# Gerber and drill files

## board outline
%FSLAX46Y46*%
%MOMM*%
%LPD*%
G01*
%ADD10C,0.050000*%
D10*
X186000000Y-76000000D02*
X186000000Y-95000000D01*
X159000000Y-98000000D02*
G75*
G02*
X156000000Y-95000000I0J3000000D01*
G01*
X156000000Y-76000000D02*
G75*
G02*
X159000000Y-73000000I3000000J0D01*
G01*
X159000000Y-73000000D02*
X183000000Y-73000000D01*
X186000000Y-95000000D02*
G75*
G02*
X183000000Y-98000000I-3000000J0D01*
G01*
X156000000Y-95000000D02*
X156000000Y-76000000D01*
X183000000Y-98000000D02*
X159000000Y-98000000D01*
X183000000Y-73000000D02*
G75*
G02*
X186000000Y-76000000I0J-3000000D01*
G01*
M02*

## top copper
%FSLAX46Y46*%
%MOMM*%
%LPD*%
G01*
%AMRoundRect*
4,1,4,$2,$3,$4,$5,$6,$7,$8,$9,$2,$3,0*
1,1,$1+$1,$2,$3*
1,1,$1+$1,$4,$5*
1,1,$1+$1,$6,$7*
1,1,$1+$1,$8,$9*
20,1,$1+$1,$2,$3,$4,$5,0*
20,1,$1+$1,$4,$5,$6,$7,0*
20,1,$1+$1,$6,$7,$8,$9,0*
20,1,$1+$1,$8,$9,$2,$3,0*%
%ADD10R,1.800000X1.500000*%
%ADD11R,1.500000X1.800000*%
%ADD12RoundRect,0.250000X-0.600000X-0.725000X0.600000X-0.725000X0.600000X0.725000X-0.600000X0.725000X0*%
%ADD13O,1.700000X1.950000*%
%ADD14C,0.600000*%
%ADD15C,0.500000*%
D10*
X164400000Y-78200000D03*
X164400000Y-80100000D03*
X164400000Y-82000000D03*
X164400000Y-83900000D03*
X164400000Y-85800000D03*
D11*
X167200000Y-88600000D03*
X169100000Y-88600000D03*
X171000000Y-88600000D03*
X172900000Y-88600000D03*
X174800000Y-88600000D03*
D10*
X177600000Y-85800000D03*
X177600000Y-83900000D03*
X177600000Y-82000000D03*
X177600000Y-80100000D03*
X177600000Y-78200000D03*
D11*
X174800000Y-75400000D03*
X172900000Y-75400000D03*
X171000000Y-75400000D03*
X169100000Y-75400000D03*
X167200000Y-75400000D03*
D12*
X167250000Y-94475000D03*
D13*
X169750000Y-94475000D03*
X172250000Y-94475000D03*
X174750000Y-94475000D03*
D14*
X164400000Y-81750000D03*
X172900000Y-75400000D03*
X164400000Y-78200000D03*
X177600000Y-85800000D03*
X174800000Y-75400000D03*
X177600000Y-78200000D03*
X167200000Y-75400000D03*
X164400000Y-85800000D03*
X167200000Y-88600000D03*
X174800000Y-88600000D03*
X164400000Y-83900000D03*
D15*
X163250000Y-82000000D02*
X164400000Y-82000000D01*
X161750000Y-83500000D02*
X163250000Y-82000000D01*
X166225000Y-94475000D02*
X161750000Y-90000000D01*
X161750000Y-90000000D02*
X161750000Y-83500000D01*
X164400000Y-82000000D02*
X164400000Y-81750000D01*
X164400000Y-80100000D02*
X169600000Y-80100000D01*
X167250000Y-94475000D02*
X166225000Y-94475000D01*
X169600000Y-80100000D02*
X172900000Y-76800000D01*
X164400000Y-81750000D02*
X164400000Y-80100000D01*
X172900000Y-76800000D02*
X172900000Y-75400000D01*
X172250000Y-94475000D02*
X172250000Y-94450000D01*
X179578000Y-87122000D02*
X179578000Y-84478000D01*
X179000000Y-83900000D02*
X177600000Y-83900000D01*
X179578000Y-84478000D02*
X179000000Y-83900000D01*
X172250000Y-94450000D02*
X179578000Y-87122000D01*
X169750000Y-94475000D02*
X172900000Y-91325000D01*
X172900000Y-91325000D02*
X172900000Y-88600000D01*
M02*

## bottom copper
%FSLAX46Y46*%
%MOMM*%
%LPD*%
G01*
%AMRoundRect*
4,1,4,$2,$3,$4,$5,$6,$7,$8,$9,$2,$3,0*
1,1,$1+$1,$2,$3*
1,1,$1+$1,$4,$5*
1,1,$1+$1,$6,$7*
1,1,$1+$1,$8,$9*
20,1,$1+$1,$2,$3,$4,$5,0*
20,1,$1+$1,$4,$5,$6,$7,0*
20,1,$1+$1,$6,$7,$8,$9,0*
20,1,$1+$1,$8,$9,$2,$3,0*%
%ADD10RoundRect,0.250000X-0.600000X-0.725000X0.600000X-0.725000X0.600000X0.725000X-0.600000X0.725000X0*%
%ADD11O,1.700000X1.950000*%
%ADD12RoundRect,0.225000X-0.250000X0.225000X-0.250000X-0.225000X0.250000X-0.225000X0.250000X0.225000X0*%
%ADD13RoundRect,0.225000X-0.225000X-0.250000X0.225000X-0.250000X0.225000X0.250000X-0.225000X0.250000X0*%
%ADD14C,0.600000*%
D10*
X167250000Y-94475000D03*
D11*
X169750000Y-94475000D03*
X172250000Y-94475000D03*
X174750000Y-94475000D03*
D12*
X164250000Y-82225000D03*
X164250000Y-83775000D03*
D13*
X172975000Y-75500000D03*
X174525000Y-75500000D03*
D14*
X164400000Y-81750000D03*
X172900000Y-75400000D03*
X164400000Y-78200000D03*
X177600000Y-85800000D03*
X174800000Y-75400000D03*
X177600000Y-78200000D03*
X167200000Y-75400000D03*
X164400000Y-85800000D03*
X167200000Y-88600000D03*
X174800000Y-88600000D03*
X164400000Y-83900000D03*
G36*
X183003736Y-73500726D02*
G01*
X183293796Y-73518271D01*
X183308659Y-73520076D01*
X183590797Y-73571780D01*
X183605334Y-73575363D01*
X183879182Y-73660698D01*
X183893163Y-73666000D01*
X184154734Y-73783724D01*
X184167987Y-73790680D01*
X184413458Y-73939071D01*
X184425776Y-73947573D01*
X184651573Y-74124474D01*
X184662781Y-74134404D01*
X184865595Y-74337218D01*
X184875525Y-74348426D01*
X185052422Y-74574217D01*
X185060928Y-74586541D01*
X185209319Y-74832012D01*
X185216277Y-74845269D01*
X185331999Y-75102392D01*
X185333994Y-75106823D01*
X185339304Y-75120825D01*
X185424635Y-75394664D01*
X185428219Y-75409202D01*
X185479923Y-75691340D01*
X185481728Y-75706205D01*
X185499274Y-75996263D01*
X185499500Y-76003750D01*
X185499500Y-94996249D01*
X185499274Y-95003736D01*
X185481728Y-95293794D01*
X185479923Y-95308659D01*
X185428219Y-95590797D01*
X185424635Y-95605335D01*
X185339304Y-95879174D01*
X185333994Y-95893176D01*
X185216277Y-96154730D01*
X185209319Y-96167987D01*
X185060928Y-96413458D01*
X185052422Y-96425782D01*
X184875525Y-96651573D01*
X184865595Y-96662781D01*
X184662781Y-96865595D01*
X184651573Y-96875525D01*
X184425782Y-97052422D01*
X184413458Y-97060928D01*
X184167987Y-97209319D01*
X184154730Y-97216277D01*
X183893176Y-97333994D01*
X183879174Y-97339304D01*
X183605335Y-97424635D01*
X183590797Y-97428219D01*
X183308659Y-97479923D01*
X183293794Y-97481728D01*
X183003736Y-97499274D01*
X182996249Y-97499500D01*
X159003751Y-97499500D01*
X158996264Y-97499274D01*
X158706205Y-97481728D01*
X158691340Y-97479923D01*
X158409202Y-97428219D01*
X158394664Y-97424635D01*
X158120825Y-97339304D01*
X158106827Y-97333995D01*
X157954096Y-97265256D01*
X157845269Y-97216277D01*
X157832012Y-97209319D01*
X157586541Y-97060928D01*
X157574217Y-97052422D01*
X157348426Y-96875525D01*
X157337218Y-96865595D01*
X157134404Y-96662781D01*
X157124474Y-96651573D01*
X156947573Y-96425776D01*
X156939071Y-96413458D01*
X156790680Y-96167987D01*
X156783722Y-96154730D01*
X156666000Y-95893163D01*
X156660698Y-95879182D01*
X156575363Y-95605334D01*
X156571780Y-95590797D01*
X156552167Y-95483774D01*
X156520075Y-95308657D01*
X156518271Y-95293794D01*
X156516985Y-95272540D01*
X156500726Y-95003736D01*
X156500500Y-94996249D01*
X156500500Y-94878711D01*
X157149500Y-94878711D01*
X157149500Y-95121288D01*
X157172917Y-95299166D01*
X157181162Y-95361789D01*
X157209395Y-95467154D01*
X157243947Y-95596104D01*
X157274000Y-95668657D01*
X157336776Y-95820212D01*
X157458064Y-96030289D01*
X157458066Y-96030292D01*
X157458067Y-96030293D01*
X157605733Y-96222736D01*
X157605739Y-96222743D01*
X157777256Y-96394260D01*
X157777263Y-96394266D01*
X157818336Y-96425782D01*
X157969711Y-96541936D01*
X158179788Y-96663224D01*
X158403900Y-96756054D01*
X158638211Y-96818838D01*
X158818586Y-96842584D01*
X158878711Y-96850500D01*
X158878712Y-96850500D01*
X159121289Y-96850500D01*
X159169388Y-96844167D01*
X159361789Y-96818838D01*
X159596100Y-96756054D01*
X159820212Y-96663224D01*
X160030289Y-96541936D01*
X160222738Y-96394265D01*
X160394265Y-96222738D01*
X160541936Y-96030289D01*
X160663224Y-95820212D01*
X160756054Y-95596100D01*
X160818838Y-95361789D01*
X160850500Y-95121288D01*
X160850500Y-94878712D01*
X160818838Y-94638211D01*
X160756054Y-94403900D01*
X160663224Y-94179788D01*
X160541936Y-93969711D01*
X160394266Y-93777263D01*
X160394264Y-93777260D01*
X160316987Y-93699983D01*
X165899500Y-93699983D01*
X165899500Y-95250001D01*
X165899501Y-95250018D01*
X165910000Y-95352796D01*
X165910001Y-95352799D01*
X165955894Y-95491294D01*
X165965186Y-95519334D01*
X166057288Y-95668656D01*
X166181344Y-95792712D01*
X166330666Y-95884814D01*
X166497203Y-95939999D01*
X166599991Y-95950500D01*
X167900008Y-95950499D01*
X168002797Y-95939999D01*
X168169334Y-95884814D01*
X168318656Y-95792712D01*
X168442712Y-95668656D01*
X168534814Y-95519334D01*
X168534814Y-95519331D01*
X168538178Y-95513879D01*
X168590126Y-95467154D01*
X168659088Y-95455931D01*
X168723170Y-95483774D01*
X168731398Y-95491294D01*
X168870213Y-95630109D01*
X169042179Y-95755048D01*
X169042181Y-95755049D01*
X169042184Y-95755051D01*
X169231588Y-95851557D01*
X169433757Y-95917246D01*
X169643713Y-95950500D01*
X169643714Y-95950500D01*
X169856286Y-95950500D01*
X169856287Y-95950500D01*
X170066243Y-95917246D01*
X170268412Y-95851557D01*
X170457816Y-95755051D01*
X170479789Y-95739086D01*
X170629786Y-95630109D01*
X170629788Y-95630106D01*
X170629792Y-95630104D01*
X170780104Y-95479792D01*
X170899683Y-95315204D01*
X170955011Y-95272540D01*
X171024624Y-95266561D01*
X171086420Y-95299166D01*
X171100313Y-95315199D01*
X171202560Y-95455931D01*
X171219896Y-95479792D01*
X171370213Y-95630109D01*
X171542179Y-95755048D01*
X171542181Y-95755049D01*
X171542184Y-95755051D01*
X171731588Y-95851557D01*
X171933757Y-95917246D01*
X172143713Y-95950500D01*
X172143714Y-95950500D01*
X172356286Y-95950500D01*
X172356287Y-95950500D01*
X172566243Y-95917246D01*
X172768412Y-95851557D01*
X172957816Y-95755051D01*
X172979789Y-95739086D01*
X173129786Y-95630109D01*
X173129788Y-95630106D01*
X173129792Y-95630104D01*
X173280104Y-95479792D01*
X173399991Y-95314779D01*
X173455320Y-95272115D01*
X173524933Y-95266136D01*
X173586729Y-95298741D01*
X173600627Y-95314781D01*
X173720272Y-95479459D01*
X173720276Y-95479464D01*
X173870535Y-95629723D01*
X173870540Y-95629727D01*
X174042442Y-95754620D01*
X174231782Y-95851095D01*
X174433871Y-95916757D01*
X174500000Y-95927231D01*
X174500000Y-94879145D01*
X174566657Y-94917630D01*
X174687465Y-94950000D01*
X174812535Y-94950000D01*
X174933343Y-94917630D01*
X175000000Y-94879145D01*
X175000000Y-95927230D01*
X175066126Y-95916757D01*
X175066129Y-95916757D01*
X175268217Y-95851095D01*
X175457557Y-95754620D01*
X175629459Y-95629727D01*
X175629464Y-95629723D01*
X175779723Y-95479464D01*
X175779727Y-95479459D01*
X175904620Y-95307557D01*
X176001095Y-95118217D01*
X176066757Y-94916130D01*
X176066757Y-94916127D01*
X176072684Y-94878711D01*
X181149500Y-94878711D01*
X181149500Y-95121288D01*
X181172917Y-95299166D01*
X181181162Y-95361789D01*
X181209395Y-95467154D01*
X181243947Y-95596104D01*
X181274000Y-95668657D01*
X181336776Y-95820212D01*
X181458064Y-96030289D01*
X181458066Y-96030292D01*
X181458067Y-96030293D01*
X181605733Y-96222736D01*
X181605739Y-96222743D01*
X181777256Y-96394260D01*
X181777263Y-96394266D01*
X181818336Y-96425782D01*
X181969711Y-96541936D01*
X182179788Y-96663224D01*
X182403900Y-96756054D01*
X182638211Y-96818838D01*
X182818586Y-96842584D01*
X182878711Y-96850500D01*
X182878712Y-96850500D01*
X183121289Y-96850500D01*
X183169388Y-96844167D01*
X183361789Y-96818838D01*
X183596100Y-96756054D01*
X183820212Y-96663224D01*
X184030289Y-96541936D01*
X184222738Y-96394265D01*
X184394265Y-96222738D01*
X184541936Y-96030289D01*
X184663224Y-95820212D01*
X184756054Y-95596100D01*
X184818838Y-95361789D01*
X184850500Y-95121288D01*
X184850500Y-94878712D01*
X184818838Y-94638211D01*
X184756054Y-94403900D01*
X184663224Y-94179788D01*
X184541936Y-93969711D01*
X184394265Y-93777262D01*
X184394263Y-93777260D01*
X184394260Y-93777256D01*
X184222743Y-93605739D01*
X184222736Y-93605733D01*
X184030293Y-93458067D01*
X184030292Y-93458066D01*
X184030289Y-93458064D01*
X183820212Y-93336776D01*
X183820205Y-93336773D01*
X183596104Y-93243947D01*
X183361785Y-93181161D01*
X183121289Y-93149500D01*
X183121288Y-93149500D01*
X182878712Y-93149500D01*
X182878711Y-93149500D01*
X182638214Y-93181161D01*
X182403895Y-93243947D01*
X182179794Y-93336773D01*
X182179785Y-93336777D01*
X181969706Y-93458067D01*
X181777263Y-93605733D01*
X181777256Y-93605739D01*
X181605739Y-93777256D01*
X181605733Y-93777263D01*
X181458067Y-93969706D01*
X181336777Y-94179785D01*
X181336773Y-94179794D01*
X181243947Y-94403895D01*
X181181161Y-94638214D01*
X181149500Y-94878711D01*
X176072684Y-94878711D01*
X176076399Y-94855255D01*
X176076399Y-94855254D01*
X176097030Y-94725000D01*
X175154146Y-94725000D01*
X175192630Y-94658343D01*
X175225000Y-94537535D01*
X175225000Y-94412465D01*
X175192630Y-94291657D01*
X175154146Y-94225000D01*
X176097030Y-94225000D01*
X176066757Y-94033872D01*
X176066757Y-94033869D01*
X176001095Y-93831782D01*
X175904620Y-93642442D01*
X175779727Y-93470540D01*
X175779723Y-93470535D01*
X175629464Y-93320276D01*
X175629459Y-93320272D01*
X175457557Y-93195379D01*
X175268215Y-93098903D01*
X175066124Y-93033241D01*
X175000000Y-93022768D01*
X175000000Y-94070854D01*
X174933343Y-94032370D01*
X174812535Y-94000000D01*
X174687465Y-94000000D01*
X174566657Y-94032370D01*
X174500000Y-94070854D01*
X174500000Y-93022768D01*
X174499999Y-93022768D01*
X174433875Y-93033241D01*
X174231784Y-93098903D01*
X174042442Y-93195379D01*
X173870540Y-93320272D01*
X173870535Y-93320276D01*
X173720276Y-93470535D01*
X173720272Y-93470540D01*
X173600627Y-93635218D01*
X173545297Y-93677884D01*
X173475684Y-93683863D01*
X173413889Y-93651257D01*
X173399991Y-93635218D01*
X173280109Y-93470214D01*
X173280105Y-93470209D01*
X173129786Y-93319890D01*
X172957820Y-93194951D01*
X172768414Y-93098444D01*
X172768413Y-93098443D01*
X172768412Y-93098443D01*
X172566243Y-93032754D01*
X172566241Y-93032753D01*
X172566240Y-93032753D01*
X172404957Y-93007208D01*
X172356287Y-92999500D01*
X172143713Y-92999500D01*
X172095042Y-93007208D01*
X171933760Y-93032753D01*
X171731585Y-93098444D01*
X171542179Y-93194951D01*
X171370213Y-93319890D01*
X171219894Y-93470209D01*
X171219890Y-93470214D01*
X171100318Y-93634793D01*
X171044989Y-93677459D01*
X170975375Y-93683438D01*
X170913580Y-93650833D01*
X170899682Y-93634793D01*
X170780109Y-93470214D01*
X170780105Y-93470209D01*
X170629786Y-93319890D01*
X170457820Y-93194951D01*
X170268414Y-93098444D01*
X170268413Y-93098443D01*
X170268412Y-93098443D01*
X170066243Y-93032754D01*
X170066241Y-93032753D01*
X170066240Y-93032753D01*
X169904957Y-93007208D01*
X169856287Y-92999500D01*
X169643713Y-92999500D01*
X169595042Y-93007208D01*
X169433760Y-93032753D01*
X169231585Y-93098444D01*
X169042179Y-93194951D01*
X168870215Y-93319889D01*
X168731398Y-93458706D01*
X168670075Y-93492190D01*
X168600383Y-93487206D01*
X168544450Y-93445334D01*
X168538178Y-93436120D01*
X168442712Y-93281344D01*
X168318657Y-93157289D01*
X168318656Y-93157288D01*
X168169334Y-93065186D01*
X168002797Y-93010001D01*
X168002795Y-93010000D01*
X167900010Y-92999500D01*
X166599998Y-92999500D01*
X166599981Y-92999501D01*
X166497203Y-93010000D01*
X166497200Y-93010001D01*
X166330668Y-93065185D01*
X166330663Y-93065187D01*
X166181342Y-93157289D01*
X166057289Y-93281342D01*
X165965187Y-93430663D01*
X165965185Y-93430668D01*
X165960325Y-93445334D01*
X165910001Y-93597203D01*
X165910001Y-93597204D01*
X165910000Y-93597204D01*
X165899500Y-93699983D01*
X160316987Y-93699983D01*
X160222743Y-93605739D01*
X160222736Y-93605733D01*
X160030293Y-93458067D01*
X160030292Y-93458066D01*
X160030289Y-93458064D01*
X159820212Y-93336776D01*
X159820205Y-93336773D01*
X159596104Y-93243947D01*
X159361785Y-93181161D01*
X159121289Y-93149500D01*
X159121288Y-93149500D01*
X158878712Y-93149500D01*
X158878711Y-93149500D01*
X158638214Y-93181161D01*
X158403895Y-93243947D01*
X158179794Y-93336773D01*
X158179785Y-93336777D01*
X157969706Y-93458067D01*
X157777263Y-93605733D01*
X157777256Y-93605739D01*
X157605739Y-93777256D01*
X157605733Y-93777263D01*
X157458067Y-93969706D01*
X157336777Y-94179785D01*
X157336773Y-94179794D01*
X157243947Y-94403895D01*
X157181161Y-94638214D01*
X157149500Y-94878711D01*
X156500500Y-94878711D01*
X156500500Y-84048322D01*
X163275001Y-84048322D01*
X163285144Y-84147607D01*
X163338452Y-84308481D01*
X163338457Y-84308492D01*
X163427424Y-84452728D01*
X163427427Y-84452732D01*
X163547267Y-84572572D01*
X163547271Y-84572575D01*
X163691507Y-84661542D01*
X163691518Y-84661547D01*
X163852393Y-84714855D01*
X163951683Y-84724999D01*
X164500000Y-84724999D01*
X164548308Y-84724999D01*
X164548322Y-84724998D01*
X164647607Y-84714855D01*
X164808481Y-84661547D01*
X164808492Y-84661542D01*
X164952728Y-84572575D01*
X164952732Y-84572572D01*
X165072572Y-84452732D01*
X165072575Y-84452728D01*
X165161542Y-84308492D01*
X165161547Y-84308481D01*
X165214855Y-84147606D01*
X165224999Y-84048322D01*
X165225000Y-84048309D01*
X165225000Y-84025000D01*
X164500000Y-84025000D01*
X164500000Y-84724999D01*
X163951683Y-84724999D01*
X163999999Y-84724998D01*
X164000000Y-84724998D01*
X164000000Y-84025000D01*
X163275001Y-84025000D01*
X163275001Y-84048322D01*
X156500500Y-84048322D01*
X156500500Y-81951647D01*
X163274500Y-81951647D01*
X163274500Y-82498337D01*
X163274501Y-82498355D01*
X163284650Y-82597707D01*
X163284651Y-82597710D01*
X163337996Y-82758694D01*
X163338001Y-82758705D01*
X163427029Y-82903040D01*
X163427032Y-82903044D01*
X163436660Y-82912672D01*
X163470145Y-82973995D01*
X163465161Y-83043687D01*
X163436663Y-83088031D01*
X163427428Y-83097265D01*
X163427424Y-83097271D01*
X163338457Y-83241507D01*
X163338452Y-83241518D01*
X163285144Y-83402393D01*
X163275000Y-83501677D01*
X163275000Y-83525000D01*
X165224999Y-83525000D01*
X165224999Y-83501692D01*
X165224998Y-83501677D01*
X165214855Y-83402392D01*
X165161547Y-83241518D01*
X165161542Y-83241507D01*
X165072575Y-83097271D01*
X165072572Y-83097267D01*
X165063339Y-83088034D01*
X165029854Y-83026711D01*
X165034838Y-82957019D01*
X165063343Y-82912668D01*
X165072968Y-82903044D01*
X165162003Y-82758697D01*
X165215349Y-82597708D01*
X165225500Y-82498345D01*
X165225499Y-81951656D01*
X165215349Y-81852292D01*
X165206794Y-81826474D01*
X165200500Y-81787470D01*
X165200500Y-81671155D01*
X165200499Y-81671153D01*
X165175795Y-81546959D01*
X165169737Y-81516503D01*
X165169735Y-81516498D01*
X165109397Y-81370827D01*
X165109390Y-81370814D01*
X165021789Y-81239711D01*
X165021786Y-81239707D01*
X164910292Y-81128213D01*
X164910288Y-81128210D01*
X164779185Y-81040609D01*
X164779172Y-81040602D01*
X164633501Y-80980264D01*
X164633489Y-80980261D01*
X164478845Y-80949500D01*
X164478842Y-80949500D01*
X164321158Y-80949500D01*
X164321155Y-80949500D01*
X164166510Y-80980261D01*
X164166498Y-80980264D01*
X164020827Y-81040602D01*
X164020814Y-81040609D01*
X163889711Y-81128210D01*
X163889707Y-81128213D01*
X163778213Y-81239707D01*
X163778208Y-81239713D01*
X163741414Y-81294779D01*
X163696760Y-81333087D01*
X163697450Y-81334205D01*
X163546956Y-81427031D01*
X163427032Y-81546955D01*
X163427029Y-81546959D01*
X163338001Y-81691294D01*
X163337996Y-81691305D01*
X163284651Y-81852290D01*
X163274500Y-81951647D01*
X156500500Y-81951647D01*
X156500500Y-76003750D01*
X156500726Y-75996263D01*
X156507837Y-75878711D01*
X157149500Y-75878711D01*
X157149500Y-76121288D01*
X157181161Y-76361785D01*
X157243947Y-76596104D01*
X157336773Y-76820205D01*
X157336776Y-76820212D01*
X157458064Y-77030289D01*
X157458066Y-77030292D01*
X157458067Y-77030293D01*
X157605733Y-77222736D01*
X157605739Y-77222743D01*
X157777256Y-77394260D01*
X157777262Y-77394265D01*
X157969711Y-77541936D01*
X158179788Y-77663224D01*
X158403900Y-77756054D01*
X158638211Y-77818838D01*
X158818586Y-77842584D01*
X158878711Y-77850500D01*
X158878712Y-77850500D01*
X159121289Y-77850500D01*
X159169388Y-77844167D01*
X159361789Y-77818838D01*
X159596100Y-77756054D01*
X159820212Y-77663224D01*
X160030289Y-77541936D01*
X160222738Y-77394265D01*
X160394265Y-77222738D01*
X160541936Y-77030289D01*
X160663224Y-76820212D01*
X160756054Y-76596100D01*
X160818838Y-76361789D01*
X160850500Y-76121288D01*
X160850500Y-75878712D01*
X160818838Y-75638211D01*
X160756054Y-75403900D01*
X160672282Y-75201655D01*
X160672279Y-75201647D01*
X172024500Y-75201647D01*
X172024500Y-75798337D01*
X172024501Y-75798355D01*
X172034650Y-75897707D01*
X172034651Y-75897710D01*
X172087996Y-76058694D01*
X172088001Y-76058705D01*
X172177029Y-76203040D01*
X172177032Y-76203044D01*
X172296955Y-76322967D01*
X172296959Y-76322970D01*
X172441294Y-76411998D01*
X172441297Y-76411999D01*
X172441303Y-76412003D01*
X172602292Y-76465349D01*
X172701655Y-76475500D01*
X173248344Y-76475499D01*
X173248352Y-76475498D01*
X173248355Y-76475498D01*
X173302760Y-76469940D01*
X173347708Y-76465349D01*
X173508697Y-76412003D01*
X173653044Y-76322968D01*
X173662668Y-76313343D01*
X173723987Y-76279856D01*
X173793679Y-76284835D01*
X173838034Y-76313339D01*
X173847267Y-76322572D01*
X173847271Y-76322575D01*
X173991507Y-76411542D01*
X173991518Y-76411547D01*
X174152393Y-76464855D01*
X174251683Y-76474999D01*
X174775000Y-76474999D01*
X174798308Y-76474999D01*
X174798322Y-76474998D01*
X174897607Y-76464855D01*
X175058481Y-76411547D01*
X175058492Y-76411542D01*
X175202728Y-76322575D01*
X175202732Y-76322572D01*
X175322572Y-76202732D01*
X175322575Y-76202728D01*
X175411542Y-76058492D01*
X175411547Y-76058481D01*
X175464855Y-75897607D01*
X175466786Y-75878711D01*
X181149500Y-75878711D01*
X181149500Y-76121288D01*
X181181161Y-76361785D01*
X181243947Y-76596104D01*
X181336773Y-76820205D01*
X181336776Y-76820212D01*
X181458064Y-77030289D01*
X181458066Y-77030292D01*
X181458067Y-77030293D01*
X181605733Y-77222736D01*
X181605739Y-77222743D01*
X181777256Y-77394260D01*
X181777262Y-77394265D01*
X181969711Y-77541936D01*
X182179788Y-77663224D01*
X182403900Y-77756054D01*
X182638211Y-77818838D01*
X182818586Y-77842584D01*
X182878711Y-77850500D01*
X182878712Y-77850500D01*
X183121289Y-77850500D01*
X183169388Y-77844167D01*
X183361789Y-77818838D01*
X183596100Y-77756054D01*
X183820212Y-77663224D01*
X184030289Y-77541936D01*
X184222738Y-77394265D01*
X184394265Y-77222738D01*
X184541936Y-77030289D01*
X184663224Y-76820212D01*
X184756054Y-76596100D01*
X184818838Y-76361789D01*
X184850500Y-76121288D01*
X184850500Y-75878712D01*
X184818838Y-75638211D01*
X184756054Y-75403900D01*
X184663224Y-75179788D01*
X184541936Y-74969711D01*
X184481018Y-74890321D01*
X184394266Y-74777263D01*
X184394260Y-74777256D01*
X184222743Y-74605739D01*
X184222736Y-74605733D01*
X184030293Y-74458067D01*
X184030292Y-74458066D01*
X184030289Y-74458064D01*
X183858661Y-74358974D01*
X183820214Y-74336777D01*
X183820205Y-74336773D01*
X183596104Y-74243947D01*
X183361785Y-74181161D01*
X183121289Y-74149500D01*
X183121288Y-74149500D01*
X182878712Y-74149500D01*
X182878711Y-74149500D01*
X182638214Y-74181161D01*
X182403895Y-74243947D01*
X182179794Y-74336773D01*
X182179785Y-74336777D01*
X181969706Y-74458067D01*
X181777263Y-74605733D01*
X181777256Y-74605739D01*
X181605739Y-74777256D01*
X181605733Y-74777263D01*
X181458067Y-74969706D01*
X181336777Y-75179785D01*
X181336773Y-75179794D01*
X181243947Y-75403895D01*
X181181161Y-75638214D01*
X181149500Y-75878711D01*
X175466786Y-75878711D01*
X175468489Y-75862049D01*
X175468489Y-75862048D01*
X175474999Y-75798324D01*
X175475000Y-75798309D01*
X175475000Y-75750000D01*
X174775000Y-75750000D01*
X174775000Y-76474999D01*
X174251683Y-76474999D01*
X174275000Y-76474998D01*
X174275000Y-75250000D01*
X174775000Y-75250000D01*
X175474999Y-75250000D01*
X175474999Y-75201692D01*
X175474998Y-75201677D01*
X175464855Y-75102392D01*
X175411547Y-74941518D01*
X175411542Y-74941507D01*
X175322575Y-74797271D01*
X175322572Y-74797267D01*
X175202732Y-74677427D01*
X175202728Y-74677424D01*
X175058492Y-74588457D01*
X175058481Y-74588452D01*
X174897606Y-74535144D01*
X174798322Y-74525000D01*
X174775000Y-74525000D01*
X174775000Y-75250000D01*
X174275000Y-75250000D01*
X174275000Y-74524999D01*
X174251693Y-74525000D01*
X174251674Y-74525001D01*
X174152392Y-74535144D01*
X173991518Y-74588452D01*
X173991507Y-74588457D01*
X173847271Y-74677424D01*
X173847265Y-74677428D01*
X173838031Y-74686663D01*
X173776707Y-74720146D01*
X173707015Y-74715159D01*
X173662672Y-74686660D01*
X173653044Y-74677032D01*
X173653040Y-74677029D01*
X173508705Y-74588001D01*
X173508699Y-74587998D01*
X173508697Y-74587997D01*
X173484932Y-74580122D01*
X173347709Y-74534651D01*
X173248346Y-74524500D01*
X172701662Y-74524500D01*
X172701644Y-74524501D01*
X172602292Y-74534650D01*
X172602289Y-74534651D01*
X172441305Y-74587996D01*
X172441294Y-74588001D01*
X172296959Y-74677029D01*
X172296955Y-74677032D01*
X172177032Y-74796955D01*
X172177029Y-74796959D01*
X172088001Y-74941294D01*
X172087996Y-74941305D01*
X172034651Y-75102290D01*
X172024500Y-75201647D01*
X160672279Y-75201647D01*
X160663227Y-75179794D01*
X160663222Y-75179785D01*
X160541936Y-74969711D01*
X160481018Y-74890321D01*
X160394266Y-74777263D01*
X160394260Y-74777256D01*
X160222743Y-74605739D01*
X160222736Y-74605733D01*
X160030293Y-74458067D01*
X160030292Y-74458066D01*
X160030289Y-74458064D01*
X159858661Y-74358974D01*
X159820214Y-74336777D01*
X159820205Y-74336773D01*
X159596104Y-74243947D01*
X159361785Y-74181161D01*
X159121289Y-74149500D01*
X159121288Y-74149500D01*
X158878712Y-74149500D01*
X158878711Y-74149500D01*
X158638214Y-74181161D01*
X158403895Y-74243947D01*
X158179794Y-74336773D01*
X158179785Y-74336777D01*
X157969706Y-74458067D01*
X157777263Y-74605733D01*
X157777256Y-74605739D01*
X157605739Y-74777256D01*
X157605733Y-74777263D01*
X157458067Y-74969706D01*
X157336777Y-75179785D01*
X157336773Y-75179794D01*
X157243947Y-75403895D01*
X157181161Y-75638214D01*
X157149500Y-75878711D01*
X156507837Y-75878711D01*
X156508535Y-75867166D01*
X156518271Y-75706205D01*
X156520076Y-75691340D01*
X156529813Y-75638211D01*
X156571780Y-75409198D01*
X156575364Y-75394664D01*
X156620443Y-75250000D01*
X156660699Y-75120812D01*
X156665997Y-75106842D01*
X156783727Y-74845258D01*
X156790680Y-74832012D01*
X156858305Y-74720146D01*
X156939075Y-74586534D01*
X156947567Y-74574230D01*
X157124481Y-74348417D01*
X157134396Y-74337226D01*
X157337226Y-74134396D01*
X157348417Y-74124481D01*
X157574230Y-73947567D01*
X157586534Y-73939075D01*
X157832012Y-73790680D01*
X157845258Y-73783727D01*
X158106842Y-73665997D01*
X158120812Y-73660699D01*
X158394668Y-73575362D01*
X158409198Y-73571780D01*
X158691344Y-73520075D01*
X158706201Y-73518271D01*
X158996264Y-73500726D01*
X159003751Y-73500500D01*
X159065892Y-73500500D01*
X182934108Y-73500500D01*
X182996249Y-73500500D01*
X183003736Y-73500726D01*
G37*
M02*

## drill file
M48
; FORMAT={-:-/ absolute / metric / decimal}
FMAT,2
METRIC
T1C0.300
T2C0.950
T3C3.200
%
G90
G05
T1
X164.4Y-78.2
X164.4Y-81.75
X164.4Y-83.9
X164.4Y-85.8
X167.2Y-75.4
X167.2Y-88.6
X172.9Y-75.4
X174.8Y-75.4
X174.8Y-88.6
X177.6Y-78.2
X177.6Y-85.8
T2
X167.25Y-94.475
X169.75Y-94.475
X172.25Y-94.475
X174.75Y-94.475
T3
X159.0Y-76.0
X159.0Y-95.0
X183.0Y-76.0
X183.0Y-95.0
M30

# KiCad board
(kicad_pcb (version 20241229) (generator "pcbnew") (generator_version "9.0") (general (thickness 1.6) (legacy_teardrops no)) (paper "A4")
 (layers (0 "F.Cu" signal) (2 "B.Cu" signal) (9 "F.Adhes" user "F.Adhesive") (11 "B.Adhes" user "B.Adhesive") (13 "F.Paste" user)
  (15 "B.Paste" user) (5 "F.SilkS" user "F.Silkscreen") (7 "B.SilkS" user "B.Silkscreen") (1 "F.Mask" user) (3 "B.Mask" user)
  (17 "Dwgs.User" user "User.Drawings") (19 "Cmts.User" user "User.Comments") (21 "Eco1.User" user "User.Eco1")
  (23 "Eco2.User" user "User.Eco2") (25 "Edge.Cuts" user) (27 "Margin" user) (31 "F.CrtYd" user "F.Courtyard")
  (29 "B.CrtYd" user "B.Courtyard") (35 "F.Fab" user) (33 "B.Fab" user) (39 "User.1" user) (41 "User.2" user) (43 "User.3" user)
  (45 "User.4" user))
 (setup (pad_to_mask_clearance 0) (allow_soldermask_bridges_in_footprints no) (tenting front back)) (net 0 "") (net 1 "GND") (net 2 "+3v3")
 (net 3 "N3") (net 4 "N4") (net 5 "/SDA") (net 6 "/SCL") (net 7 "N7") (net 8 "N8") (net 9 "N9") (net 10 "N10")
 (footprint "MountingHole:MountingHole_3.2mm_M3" (layer "F.Cu") (at 183 76)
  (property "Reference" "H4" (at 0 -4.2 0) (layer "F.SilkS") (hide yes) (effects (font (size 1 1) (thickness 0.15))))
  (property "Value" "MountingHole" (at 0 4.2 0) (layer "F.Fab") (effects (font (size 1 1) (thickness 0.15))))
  (pad "" np_thru_hole circle (at 0 0) (size 3.2 3.2) (drill 3.2) (layers "*.Cu" "*.Mask")))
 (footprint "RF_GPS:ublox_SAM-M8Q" (layer "F.Cu") (at 171 82)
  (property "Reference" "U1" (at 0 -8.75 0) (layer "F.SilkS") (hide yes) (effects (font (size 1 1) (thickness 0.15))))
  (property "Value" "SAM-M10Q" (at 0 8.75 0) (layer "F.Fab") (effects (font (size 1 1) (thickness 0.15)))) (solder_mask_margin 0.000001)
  (pad "" smd rect (at -7.1 -4.225) (size 0.72 0.58) (layers "F.Paste"))
  (pad "" smd rect (at -7.1 -3.375) (size 0.72 0.58) (layers "F.Paste"))
  (pad "" smd rect (at -7.1 -2.325) (size 0.72 0.58) (layers "F.Paste"))
  (pad "" smd rect (at -7.1 -1.475) (size 0.72 0.58) (layers "F.Paste"))
  (pad "" smd rect (at -7.1 -0.425) (size 0.72 0.58) (layers "F.Paste"))
  (pad "" smd rect (at -7.1 0.425) (size 0.72 0.58) (layers "F.Paste"))
  (pad "" smd rect (at -7.1 1.475) (size 0.72 0.58) (layers "F.Paste"))
  (pad "" smd rect (at -7.1 2.325) (size 0.72 0.58) (layers "F.Paste"))
  (pad "" smd rect (at -7.1 3.375) (size 0.72 0.58) (layers "F.Paste"))
  (pad "" smd rect (at -7.1 4.225) (size 0.72 0.58) (layers "F.Paste"))
  (pad "" smd rect (at -6.1 -4.225) (size 0.72 0.58) (layers "F.Paste"))
  (pad "" smd rect (at -6.1 -3.375) (size 0.72 0.58) (layers "F.Paste"))
  (pad "" smd rect (at -6.1 -2.325) (size 0.72 0.58) (layers "F.Paste"))
  (pad "" smd rect (at -6.1 -1.475) (size 0.72 0.58) (layers "F.Paste"))
  (pad "" smd rect (at -6.1 -0.425) (size 0.72 0.58) (layers "F.Paste"))
  (pad "" smd rect (at -6.1 0.425) (size 0.72 0.58) (layers "F.Paste"))
  (pad "" smd rect (at -6.1 1.475) (size 0.72 0.58) (layers "F.Paste"))
  (pad "" smd rect (at -6.1 2.325) (size 0.72 0.58) (layers "F.Paste"))
  (pad "" smd rect (at -6.1 3.375) (size 0.72 0.58) (layers "F.Paste"))
  (pad "" smd rect (at -6.1 4.225) (size 0.72 0.58) (layers "F.Paste"))
  (pad "" smd rect (at -4.225 -7.1) (size 0.58 0.72) (layers "F.Paste"))
  (pad "" smd rect (at -4.225 -6.1) (size 0.58 0.72) (layers "F.Paste"))
  (pad "" smd rect (at -4.225 6.1) (size 0.58 0.72) (layers "F.Paste"))
  (pad "" smd rect (at -4.225 7.1) (size 0.58 0.72) (layers "F.Paste"))
  (pad "" smd rect (at -3.375 -7.1) (size 0.58 0.72) (layers "F.Paste"))
  (pad "" smd rect (at -3.375 -6.1) (size 0.58 0.72) (layers "F.Paste"))
  (pad "" smd rect (at -3.375 6.1) (size 0.58 0.72) (layers "F.Paste"))
  (pad "" smd rect (at -3.375 7.1) (size 0.58 0.72) (layers "F.Paste"))
  (pad "" smd rect (at -2.325 -7.1) (size 0.58 0.72) (layers "F.Paste"))
  (pad "" smd rect (at -2.325 -6.1) (size 0.58 0.72) (layers "F.Paste"))
  (pad "" smd rect (at -2.325 6.1) (size 0.58 0.72) (layers "F.Paste"))
  (pad "" smd rect (at -2.325 7.1) (size 0.58 0.72) (layers "F.Paste"))
  (pad "" smd rect (at -1.475 -7.1) (size 0.58 0.72) (layers "F.Paste"))
  (pad "" smd rect (at -1.475 -6.1) (size 0.58 0.72) (layers "F.Paste"))
  (pad "" smd rect (at -1.475 6.1) (size 0.58 0.72) (layers "F.Paste"))
  (pad "" smd rect (at -1.475 7.1) (size 0.58 0.72) (layers "F.Paste"))
  (pad "" smd rect (at -0.425 -7.1) (size 0.58 0.72) (layers "F.Paste"))
  (pad "" smd rect (at -0.425 -6.1) (size 0.58 0.72) (layers "F.Paste"))
  (pad "" smd rect (at -0.425 6.1) (size 0.58 0.72) (layers "F.Paste"))
  (pad "" smd rect (at -0.425 7.1) (size 0.58 0.72) (layers "F.Paste"))
  (pad "" smd rect (at 0.425 -7.1) (size 0.58 0.72) (layers "F.Paste"))
  (pad "" smd rect (at 0.425 -6.1) (size 0.58 0.72) (layers "F.Paste"))
  (pad "" smd rect (at 0.425 6.1) (size 0.58 0.72) (layers "F.Paste"))
  (pad "" smd rect (at 0.425 7.1) (size 0.58 0.72) (layers "F.Paste"))
  (pad "" smd rect (at 1.475 -7.1) (size 0.58 0.72) (layers "F.Paste"))
  (pad "" smd rect (at 1.475 -6.1) (size 0.58 0.72) (layers "F.Paste"))
  (pad "" smd rect (at 1.475 6.1) (size 0.58 0.72) (layers "F.Paste"))
  (pad "" smd rect (at 1.475 7.1) (size 0.58 0.72) (layers "F.Paste"))
  (pad "" smd rect (at 2.325 -7.1) (size 0.58 0.72) (layers "F.Paste"))
  (pad "" smd rect (at 2.325 -6.1) (size 0.58 0.72) (layers "F.Paste"))
  (pad "" smd rect (at 2.325 6.1) (size 0.58 0.72) (layers "F.Paste"))
  (pad "" smd rect (at 2.325 7.1) (size 0.58 0.72) (layers "F.Paste"))
  (pad "" smd rect (at 3.375 -7.1) (size 0.58 0.72) (layers "F.Paste"))
  (pad "" smd rect (at 3.375 -6.1) (size 0.58 0.72) (layers "F.Paste"))
  (pad "" smd rect (at 3.375 6.1) (size 0.58 0.72) (layers "F.Paste"))
  (pad "" smd rect (at 3.375 7.1) (size 0.58 0.72) (layers "F.Paste"))
  (pad "" smd rect (at 4.225 -7.1) (size 0.58 0.72) (layers "F.Paste"))
  (pad "" smd rect (at 4.225 -6.1) (size 0.58 0.72) (layers "F.Paste"))
  (pad "" smd rect (at 4.225 6.1) (size 0.58 0.72) (layers "F.Paste"))
  (pad "" smd rect (at 4.225 7.1) (size 0.58 0.72) (layers "F.Paste"))
  (pad "" smd rect (at 6.1 -4.225) (size 0.72 0.58) (layers "F.Paste"))
  (pad "" smd rect (at 6.1 -3.375) (size 0.72 0.58) (layers "F.Paste"))
  (pad "" smd rect (at 6.1 -2.325) (size 0.72 0.58) (layers "F.Paste"))
  (pad "" smd rect (at 6.1 -1.475) (size 0.72 0.58) (layers "F.Paste"))
  (pad "" smd rect (at 6.1 -0.425) (size 0.72 0.58) (layers "F.Paste"))
  (pad "" smd rect (at 6.1 0.425) (size 0.72 0.58) (layers "F.Paste"))
  (pad "" smd rect (at 6.1 1.475) (size 0.72 0.58) (layers "F.Paste"))
  (pad "" smd rect (at 6.1 2.325) (size 0.72 0.58) (layers "F.Paste"))
  (pad "" smd rect (at 6.1 3.375) (size 0.72 0.58) (layers "F.Paste"))
  (pad "" smd rect (at 6.1 4.225) (size 0.72 0.58) (layers "F.Paste"))
  (pad "" smd rect (at 7.1 -4.225) (size 0.72 0.58) (layers "F.Paste"))
  (pad "" smd rect (at 7.1 -3.375) (size 0.72 0.58) (layers "F.Paste"))
  (pad "" smd rect (at 7.1 -2.325) (size 0.72 0.58) (layers "F.Paste"))
  (pad "" smd rect (at 7.1 -1.475) (size 0.72 0.58) (layers "F.Paste"))
  (pad "" smd rect (at 7.1 -0.425) (size 0.72 0.58) (layers "F.Paste"))
  (pad "" smd rect (at 7.1 0.425) (size 0.72 0.58) (layers "F.Paste"))
  (pad "" smd rect (at 7.1 1.475) (size 0.72 0.58) (layers "F.Paste"))
  (pad "" smd rect (at 7.1 2.325) (size 0.72 0.58) (layers "F.Paste"))
  (pad "" smd rect (at 7.1 3.375) (size 0.72 0.58) (layers "F.Paste"))
  (pad "" smd rect (at 7.1 4.225) (size 0.72 0.58) (layers "F.Paste"))
  (pad "1" smd rect (at -6.6 -3.8) (size 1.8 1.5) (layers "F.Cu" "F.Mask") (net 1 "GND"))
  (pad "2" smd rect (at -6.6 -1.9) (size 1.8 1.5) (layers "F.Cu" "F.Mask") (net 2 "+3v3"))
  (pad "3" smd rect (at -6.6 0) (size 1.8 1.5) (layers "F.Cu" "F.Mask") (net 2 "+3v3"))
  (pad "4" smd rect (at -6.6 1.9) (size 1.8 1.5) (layers "F.Cu" "F.Mask") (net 1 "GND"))
  (pad "5" smd rect (at -6.6 3.8) (size 1.8 1.5) (layers "F.Cu" "F.Mask") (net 1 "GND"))
  (pad "6" smd rect (at -3.8 6.6) (size 1.5 1.8) (layers "F.Cu" "F.Mask") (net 1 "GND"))
  (pad "7" smd rect (at -1.9 6.6) (size 1.5 1.8) (layers "F.Cu" "F.Mask") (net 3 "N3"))
  (pad "8" smd rect (at 0 6.6) (size 1.5 1.8) (layers "F.Cu" "F.Mask") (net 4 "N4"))
  (pad "9" smd rect (at 1.9 6.6) (size 1.5 1.8) (layers "F.Cu" "F.Mask") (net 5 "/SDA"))
  (pad "10" smd rect (at 3.8 6.6) (size 1.5 1.8) (layers "F.Cu" "F.Mask") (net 1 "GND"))
  (pad "11" smd rect (at 6.6 3.8) (size 1.8 1.5) (layers "F.Cu" "F.Mask") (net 1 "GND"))
  (pad "12" smd rect (at 6.6 1.9) (size 1.8 1.5) (layers "F.Cu" "F.Mask") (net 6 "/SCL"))
  (pad "13" smd rect (at 6.6 0) (size 1.8 1.5) (layers "F.Cu" "F.Mask") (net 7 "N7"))
  (pad "14" smd rect (at 6.6 -1.9) (size 1.8 1.5) (layers "F.Cu" "F.Mask") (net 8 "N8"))
  (pad "15" smd rect (at 6.6 -3.8) (size 1.8 1.5) (layers "F.Cu" "F.Mask") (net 1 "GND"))
  (pad "16" smd rect (at 3.8 -6.6) (size 1.5 1.8) (layers "F.Cu" "F.Mask") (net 1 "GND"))
  (pad "17" smd rect (at 1.9 -6.6) (size 1.5 1.8) (layers "F.Cu" "F.Mask") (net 2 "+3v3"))
  (pad "18" smd rect (at 0 -6.6) (size 1.5 1.8) (layers "F.Cu" "F.Mask") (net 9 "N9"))
  (pad "19" smd rect (at -1.9 -6.6) (size 1.5 1.8) (layers "F.Cu" "F.Mask") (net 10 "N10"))
  (pad "20" smd rect (at -3.8 -6.6) (size 1.5 1.8) (layers "F.Cu" "F.Mask") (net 1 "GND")))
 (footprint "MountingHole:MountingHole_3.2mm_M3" (layer "F.Cu") (at 183 95)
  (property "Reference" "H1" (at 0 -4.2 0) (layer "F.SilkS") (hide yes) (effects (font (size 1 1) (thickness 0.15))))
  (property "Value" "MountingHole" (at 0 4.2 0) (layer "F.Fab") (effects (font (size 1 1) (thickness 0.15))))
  (pad "" np_thru_hole circle (at 0 0) (size 3.2 3.2) (drill 3.2) (layers "*.Cu" "*.Mask")))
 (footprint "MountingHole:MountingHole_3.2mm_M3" (layer "F.Cu") (at 159 76)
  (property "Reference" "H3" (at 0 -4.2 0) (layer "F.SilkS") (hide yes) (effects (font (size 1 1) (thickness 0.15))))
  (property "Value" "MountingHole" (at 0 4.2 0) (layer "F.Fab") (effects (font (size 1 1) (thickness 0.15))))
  (pad "" np_thru_hole circle (at 0 0) (size 3.2 3.2) (drill 3.2) (layers "*.Cu" "*.Mask")))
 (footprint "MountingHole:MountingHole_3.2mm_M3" (layer "F.Cu") (at 159 95)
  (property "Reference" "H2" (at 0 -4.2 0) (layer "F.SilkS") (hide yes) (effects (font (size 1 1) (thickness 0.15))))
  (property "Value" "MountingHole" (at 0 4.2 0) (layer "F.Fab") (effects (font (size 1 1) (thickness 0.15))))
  (pad "" np_thru_hole circle (at 0 0) (size 3.2 3.2) (drill 3.2) (layers "*.Cu" "*.Mask")))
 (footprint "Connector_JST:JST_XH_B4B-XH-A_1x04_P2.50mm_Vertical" (layer "F.Cu") (at 167.25 94.475)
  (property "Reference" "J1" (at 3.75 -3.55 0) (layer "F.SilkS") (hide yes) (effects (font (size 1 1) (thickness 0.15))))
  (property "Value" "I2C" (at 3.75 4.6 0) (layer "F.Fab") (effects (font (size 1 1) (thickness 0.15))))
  (pad "1" thru_hole roundrect (at 0 0) (size 1.7 1.95) (drill 0.95) (layers "*.Cu" "*.Mask") (remove_unused_layers no)
   (roundrect_rratio 0.147059) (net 2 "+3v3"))
  (pad "2" thru_hole oval (at 2.5 0) (size 1.7 1.95) (drill 0.95) (layers "*.Cu" "*.Mask") (remove_unused_layers no) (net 5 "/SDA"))
  (pad "3" thru_hole oval (at 5 0) (size 1.7 1.95) (drill 0.95) (layers "*.Cu" "*.Mask") (remove_unused_layers no) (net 6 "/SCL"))
  (pad "4" thru_hole oval (at 7.5 0) (size 1.7 1.95) (drill 0.95) (layers "*.Cu" "*.Mask") (remove_unused_layers no) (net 1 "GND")))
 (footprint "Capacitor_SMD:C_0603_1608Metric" (layer "B.Cu") (at 164.25 83 -90)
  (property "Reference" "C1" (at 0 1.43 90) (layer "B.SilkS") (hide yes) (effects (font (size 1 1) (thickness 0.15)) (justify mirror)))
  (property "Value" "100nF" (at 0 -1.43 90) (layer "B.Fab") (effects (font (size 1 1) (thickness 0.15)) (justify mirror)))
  (pad "1" smd roundrect (at -0.775 0 270) (size 0.9 0.95) (layers "B.Cu" "B.Mask" "B.Paste") (roundrect_rratio 0.25) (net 2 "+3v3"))
  (pad "2" smd roundrect (at 0.775 0 270) (size 0.9 0.95) (layers "B.Cu" "B.Mask" "B.Paste") (roundrect_rratio 0.25) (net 1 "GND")))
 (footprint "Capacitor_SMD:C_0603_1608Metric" (layer "B.Cu") (at 173.75 75.5)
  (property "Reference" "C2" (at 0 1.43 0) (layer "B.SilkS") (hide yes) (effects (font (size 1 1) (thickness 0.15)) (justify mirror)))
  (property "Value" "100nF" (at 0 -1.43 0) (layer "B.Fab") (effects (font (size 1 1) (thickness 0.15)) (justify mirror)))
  (pad "1" smd roundrect (at -0.775 0) (size 0.9 0.95) (layers "B.Cu" "B.Mask" "B.Paste") (roundrect_rratio 0.25) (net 2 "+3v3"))
  (pad "2" smd roundrect (at 0.775 0) (size 0.9 0.95) (layers "B.Cu" "B.Mask" "B.Paste") (roundrect_rratio 0.25) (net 1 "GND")))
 (gr_line (start 186 76) (end 186 95) (stroke (width 0.05) (type default)) (layer "Edge.Cuts"))
 (gr_arc (start 159 98) (mid 156.87868 97.12132) (end 156 95) (stroke (width 0.05) (type default)) (layer "Edge.Cuts"))
 (gr_arc (start 156 76) (mid 156.87868 73.87868) (end 159 73) (stroke (width 0.05) (type default)) (layer "Edge.Cuts"))
 (gr_line (start 159 73) (end 183 73) (stroke (width 0.05) (type default)) (layer "Edge.Cuts"))
 (gr_arc (start 186 95) (mid 185.12132 97.12132) (end 183 98) (stroke (width 0.05) (type default)) (layer "Edge.Cuts"))
 (gr_line (start 156 95) (end 156 76) (stroke (width 0.05) (type default)) (layer "Edge.Cuts"))
 (gr_line (start 183 98) (end 159 98) (stroke (width 0.05) (type default)) (layer "Edge.Cuts"))
 (gr_arc (start 183 73) (mid 185.12132 73.87868) (end 186 76) (stroke (width 0.05) (type default)) (layer "Edge.Cuts"))
 (segment (start 163.25 82) (end 164.4 82) (width 0.5) (layer "F.Cu") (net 2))
 (segment (start 161.75 83.5) (end 163.25 82) (width 0.5) (layer "F.Cu") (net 2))
 (segment (start 166.225 94.475) (end 161.75 90) (width 0.5) (layer "F.Cu") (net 2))
 (segment (start 161.75 90) (end 161.75 83.5) (width 0.5) (layer "F.Cu") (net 2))
 (segment (start 164.4 82) (end 164.4 81.75) (width 0.5) (layer "F.Cu") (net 2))
 (segment (start 164.4 80.1) (end 169.6 80.1) (width 0.5) (layer "F.Cu") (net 2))
 (segment (start 167.25 94.475) (end 166.225 94.475) (width 0.5) (layer "F.Cu") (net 2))
 (segment (start 169.6 80.1) (end 172.9 76.8) (width 0.5) (layer "F.Cu") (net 2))
 (segment (start 164.4 81.75) (end 164.4 80.1) (width 0.5) (layer "F.Cu") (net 2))
 (segment (start 172.9 76.8) (end 172.9 75.4) (width 0.5) (layer "F.Cu") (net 2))
 (via (at 164.4 81.75) (size 0.6) (drill 0.3) (layers "F.Cu" "B.Cu") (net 2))
 (via (at 172.9 75.4) (size 0.6) (drill 0.3) (layers "F.Cu" "B.Cu") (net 2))
 (via (at 164.4 78.2) (size 0.6) (drill 0.3) (layers "F.Cu" "B.Cu") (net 1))
 (via (at 177.6 85.8) (size 0.6) (drill 0.3) (layers "F.Cu" "B.Cu") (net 1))
 (via (at 174.8 75.4) (size 0.6) (drill 0.3) (layers "F.Cu" "B.Cu") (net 1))
 (via (at 177.6 78.2) (size 0.6) (drill 0.3) (layers "F.Cu" "B.Cu") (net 1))
 (via (at 167.2 75.4) (size 0.6) (drill 0.3) (layers "F.Cu" "B.Cu") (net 1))
 (via (at 164.4 85.8) (size 0.6) (drill 0.3) (layers "F.Cu" "B.Cu") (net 1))
 (via (at 167.2 88.6) (size 0.6) (drill 0.3) (layers "F.Cu" "B.Cu") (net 1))
 (via (at 174.8 88.6) (size 0.6) (drill 0.3) (layers "F.Cu" "B.Cu") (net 1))
 (via (at 164.4 83.9) (size 0.6) (drill 0.3) (layers "F.Cu" "B.Cu") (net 1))
 (segment (start 172.25 94.475) (end 172.25 94.45) (width 0.5) (layer "F.Cu") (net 6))
 (segment (start 179.578 87.122) (end 179.578 84.478) (width 0.5) (layer "F.Cu") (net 6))
 (segment (start 179 83.9) (end 177.6 83.9) (width 0.5) (layer "F.Cu") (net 6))
 (segment (start 179.578 84.478) (end 179 83.9) (width 0.5) (layer "F.Cu") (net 6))
 (segment (start 172.25 94.45) (end 179.578 87.122) (width 0.5) (layer "F.Cu") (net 6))
 (segment (start 169.75 94.475) (end 172.9 91.325) (width 0.5) (layer "F.Cu") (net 5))
 (segment (start 172.9 91.325) (end 172.9 88.6) (width 0.5) (layer "F.Cu") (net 5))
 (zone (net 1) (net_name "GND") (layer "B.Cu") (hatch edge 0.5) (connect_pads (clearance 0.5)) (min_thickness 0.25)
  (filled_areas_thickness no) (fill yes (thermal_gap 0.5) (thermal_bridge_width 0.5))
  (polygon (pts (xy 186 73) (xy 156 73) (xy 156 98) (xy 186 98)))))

